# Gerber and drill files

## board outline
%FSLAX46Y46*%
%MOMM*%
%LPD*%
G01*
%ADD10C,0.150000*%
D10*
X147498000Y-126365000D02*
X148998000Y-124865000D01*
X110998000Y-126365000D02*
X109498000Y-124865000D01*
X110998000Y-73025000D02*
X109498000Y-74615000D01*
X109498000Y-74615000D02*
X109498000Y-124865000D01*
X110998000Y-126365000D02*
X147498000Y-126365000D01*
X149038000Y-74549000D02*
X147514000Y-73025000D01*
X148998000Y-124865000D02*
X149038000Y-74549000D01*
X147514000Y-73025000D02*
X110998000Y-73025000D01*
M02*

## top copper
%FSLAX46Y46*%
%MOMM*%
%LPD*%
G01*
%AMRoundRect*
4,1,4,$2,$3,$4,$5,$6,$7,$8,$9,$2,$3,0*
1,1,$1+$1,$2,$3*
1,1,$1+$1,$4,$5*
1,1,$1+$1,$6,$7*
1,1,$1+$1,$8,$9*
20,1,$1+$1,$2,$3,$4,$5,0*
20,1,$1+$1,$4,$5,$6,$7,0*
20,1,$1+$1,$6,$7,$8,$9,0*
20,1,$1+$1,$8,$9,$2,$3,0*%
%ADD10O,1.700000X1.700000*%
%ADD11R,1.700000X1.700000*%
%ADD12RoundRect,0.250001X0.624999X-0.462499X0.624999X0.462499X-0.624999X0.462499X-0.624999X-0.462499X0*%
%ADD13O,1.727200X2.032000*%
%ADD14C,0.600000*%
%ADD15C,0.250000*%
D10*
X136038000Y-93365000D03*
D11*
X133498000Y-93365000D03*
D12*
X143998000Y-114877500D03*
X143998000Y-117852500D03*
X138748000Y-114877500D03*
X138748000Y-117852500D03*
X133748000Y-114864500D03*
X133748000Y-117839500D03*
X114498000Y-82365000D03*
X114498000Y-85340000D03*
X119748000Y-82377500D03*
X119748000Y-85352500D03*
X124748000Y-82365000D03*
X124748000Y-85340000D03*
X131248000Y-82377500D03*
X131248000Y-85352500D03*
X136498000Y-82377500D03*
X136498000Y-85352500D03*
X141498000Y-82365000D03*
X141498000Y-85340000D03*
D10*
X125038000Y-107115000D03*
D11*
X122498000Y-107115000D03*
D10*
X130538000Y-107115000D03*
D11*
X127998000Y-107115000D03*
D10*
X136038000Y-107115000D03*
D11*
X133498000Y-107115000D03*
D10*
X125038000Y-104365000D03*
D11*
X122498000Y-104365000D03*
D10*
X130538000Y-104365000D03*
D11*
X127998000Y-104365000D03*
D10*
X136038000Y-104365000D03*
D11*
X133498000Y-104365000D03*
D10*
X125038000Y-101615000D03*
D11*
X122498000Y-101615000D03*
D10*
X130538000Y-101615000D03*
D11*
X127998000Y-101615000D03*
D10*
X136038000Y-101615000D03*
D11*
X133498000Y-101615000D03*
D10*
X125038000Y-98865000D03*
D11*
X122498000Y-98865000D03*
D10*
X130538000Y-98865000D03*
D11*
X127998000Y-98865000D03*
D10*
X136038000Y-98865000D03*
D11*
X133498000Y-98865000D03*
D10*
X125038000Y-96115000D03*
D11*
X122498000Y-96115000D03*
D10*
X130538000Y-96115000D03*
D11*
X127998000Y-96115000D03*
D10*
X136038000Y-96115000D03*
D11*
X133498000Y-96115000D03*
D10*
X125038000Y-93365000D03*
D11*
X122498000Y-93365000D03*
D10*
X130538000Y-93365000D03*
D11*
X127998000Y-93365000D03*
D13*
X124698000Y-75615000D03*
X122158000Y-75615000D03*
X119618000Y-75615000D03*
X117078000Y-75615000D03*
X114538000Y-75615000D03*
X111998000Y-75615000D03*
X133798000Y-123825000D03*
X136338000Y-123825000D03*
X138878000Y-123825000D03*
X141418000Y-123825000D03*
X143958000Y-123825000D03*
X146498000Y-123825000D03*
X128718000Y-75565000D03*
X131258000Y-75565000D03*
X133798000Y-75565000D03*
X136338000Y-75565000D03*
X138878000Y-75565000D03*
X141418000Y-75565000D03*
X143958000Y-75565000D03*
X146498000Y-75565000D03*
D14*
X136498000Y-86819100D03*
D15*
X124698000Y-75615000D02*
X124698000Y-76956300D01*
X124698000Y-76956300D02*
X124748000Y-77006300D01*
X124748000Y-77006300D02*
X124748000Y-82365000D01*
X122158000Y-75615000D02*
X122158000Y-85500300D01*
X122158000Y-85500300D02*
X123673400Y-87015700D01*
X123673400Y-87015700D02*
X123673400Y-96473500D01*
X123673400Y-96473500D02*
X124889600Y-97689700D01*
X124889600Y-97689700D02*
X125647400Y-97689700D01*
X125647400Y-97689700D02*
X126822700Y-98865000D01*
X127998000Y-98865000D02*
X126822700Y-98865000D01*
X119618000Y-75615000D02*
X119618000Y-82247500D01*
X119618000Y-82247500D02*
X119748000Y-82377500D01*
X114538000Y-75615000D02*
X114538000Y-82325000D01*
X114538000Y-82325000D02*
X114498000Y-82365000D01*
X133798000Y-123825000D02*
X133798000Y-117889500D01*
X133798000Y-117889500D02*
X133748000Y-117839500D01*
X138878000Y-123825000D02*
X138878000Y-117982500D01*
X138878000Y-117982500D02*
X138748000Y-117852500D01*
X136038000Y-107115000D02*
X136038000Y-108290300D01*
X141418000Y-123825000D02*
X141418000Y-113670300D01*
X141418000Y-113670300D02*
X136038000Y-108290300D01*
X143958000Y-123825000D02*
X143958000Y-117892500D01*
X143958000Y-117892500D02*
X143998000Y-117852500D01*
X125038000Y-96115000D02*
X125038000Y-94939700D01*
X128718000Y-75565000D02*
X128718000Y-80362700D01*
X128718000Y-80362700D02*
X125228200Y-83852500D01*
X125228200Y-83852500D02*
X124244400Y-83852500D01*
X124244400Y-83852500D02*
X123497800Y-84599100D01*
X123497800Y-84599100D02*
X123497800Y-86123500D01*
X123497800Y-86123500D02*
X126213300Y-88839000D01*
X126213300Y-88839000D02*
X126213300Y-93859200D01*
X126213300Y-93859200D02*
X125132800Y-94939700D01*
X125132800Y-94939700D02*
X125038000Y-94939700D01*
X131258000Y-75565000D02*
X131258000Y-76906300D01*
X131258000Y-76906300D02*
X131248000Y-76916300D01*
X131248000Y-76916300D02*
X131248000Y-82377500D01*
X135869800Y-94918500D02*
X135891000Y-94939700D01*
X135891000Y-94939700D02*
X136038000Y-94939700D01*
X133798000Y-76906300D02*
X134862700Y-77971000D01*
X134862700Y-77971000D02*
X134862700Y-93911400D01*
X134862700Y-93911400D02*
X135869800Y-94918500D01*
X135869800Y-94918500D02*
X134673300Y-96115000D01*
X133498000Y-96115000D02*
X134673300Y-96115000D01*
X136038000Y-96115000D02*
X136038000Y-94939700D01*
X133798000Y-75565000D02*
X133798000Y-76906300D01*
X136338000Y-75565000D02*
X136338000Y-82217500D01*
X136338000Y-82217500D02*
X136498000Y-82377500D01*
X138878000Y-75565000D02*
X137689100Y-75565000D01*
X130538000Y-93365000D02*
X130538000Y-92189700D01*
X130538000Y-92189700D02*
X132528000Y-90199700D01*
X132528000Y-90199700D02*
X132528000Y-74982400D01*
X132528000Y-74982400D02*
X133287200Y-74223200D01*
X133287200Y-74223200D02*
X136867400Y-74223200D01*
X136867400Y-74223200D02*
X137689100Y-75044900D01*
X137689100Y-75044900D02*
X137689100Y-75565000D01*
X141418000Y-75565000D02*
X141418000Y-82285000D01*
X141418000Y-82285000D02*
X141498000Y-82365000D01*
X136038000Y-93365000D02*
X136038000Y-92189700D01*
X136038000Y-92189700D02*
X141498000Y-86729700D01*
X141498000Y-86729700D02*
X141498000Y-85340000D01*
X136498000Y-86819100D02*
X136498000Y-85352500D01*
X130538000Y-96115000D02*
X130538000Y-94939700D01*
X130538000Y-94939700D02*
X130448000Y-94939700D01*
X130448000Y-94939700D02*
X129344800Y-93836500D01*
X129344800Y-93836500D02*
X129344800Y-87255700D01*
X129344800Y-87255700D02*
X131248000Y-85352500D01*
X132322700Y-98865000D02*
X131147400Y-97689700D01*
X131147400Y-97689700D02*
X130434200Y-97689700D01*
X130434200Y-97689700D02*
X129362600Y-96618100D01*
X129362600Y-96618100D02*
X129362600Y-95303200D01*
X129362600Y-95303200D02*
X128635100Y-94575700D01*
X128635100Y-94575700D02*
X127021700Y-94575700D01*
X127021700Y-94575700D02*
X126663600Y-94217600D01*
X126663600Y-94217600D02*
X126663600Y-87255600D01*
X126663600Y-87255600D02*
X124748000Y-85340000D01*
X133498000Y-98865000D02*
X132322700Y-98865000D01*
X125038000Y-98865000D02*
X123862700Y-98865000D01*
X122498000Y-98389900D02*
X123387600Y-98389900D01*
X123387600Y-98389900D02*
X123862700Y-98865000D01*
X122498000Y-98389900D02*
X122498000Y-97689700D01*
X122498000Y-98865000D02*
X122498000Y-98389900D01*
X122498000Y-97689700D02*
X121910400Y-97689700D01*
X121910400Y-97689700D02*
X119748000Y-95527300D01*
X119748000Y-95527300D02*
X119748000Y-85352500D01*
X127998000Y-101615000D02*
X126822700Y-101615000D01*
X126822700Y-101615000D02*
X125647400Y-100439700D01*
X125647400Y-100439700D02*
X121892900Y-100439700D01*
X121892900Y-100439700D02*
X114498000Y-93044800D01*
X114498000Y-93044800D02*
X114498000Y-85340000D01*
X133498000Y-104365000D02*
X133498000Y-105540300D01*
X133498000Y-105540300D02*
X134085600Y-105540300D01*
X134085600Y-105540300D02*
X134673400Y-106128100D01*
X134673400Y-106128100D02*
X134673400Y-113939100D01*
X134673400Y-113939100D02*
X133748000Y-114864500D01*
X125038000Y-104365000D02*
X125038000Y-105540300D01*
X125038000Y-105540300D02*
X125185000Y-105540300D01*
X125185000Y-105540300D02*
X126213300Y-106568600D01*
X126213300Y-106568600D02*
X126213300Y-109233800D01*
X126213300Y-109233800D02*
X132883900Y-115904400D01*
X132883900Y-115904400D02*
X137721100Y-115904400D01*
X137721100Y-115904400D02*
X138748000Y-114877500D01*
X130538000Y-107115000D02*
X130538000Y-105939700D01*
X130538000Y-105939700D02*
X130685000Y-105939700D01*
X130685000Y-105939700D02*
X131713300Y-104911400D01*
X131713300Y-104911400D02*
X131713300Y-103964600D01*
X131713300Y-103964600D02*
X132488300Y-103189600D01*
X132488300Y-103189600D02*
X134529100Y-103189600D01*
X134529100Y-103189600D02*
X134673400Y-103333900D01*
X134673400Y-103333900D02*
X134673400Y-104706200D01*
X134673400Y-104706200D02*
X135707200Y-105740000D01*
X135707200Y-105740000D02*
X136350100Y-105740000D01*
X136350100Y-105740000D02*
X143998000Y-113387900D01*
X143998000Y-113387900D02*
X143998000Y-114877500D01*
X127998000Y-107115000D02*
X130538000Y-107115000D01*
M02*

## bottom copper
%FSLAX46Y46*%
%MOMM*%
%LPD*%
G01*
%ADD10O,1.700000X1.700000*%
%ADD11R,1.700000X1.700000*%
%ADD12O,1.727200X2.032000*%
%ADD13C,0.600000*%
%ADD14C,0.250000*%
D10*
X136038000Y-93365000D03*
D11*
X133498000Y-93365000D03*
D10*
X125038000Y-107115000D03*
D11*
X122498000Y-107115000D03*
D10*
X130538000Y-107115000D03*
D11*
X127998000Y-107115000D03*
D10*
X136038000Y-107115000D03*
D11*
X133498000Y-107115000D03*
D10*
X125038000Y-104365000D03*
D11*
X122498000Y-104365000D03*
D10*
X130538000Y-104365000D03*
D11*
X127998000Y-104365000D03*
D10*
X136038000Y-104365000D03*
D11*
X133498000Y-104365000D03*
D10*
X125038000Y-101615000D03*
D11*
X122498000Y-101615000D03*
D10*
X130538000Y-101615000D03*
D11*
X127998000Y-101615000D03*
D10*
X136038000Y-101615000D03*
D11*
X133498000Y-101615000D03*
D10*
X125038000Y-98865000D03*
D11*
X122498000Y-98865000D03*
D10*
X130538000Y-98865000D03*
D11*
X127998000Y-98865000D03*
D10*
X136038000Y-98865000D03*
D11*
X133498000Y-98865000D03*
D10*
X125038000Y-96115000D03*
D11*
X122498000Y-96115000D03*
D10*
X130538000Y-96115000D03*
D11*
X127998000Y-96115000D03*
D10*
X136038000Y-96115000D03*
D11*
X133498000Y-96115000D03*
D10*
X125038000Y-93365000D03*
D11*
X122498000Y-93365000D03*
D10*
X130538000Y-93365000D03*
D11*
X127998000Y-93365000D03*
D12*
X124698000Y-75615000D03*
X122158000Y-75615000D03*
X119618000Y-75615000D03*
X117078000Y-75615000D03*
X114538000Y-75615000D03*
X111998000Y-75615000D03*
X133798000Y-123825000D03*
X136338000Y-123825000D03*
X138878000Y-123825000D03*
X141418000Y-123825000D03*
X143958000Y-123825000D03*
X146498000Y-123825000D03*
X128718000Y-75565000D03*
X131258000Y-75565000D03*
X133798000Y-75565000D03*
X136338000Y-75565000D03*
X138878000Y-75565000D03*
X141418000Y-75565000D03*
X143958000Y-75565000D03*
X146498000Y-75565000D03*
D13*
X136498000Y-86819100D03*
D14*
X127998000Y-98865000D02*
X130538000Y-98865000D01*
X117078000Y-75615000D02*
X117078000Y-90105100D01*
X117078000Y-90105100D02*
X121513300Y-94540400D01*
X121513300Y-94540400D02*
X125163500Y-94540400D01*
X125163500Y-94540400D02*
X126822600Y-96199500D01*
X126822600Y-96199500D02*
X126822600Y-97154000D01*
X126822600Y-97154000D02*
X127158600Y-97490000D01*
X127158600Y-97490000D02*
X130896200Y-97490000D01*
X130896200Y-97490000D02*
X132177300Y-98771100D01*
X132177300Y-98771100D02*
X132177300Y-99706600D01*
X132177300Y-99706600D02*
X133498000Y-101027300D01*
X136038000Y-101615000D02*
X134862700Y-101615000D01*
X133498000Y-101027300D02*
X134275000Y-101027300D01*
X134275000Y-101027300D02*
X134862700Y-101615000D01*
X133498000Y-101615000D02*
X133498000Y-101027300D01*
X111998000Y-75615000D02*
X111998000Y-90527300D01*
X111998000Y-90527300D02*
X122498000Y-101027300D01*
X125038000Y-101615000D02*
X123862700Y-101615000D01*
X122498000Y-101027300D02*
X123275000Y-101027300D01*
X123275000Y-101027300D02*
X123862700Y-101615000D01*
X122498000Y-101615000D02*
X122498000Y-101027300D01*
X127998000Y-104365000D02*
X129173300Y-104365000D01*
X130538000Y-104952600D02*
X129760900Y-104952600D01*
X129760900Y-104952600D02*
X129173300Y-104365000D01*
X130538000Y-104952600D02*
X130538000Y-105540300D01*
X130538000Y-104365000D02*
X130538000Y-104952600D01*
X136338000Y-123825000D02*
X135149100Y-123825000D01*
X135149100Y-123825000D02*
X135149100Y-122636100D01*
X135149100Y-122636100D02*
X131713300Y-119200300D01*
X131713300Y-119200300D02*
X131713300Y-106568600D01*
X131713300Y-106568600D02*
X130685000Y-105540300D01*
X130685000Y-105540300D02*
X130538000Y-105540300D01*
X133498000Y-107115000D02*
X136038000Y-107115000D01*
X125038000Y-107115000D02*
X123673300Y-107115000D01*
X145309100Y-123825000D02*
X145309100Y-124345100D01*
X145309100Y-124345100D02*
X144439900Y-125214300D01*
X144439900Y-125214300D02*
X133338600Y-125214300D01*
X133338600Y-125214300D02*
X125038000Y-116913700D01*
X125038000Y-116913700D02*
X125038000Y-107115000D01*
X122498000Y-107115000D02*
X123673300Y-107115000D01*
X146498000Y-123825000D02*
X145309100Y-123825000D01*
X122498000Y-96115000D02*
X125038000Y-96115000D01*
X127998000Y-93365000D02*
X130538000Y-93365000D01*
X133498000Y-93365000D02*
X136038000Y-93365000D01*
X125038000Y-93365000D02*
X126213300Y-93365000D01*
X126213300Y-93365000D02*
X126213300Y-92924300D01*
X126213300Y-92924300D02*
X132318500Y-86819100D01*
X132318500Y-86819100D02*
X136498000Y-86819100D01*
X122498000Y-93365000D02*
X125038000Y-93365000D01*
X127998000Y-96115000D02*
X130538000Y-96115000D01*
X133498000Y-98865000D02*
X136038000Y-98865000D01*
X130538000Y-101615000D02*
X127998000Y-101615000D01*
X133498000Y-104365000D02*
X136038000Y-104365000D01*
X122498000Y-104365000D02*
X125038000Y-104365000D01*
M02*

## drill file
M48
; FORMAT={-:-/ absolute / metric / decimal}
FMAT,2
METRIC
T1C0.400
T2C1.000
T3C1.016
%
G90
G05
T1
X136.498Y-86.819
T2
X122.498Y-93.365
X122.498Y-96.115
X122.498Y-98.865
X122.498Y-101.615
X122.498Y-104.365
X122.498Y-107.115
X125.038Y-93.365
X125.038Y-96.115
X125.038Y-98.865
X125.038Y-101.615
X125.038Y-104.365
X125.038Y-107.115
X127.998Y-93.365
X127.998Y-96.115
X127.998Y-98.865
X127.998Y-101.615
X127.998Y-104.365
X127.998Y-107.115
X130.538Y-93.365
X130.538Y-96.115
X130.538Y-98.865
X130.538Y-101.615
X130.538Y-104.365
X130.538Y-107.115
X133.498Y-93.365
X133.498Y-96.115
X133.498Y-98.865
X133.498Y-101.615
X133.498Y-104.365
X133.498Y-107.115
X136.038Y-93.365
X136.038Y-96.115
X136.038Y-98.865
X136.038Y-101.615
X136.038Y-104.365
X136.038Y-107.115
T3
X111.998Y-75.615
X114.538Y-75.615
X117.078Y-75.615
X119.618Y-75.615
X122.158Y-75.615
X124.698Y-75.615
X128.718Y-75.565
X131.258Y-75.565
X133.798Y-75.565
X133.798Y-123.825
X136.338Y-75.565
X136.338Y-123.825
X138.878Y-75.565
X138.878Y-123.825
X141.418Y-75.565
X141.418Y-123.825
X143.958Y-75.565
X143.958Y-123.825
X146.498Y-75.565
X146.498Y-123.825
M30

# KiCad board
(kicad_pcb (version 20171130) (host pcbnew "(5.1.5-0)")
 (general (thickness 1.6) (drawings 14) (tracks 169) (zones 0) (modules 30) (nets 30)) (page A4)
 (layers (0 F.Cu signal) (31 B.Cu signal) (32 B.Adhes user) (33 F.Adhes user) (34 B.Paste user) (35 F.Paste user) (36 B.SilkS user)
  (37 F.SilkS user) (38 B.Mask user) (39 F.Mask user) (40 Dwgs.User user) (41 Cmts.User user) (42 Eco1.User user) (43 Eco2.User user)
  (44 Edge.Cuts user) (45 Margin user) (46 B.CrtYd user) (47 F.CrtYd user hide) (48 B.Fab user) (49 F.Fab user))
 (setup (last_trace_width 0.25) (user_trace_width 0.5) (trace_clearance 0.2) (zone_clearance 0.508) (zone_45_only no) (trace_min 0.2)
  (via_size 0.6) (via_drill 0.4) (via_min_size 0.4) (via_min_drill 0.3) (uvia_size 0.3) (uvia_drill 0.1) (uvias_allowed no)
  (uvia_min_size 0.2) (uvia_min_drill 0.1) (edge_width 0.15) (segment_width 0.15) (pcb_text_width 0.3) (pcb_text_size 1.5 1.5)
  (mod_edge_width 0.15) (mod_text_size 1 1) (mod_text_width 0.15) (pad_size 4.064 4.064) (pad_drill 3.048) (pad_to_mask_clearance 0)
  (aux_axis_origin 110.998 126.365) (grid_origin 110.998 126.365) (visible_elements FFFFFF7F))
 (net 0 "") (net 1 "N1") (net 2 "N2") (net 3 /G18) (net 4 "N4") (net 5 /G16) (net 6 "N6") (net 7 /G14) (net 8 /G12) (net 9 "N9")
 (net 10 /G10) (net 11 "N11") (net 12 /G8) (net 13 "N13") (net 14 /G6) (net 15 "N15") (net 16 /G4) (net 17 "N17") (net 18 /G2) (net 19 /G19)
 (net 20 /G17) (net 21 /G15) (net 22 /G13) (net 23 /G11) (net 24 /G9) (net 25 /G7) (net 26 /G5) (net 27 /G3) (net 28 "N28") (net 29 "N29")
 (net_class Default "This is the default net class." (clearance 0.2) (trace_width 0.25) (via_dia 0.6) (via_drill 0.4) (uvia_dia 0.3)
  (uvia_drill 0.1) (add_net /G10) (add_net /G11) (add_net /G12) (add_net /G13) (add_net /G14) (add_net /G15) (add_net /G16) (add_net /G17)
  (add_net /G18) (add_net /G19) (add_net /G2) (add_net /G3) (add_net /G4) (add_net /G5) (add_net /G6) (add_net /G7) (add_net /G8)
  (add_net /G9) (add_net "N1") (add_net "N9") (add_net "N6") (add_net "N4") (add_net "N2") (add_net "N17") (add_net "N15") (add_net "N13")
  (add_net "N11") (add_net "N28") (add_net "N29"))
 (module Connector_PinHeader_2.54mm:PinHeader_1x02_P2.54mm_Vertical (layer F.Cu) (at 133.498 93.365 90)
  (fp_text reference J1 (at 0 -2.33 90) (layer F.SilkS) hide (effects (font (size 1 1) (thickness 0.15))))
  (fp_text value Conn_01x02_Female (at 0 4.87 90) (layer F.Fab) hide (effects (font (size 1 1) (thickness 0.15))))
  (pad 2 thru_hole oval (at 0 2.54 90) (size 1.7 1.7) (drill 1) (layers *.Cu *.Mask) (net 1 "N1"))
  (pad 1 thru_hole rect (at 0 0 90) (size 1.7 1.7) (drill 1) (layers *.Cu *.Mask) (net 1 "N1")))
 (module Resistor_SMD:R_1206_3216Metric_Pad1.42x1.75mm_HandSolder (layer F.Cu) (at 143.998 116.365 90)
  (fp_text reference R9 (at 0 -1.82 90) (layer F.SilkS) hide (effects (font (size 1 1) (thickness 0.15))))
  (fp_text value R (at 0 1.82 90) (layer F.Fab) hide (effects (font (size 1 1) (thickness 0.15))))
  (pad 2 smd roundrect (at 1.4875 0 90) (size 1.425 1.75) (layers F.Cu F.Paste F.Mask) (roundrect_rratio 0.175439) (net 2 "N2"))
  (pad 1 smd roundrect (at -1.4875 0 90) (size 1.425 1.75) (layers F.Cu F.Paste F.Mask) (roundrect_rratio 0.175439) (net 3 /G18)))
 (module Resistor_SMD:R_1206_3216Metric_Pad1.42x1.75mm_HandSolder (layer F.Cu) (at 138.748 116.365 90)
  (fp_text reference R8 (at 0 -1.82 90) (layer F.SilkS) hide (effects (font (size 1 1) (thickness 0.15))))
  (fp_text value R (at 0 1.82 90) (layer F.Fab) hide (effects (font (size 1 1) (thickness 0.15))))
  (pad 2 smd roundrect (at 1.4875 0 90) (size 1.425 1.75) (layers F.Cu F.Paste F.Mask) (roundrect_rratio 0.175439) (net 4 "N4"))
  (pad 1 smd roundrect (at -1.4875 0 90) (size 1.425 1.75) (layers F.Cu F.Paste F.Mask) (roundrect_rratio 0.175439) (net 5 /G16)))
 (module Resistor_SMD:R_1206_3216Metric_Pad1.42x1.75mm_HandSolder (layer F.Cu) (at 133.748 116.352 90)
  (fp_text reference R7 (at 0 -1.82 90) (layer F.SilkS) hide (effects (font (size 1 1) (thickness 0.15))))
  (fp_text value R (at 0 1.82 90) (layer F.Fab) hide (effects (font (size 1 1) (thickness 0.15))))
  (pad 2 smd roundrect (at 1.4875 0 90) (size 1.425 1.75) (layers F.Cu F.Paste F.Mask) (roundrect_rratio 0.175439) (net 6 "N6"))
  (pad 1 smd roundrect (at -1.4875 0 90) (size 1.425 1.75) (layers F.Cu F.Paste F.Mask) (roundrect_rratio 0.175439) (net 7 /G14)))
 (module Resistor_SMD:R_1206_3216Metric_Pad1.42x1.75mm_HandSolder (layer F.Cu) (at 114.498 83.8525 90)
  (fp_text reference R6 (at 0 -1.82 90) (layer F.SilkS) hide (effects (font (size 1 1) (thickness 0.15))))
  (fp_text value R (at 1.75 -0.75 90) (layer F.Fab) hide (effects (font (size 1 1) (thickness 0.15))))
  (pad 2 smd roundrect (at 1.4875 0 90) (size 1.425 1.75) (layers F.Cu F.Paste F.Mask) (roundrect_rratio 0.175439) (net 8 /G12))
  (pad 1 smd roundrect (at -1.4875 0 90) (size 1.425 1.75) (layers F.Cu F.Paste F.Mask) (roundrect_rratio 0.175439) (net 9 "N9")))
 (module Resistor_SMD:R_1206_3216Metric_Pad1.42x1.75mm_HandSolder (layer F.Cu) (at 119.748 83.865 90)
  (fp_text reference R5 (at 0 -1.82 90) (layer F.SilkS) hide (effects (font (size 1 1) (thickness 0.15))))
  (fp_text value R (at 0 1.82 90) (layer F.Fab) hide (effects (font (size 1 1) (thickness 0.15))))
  (pad 2 smd roundrect (at 1.4875 0 90) (size 1.425 1.75) (layers F.Cu F.Paste F.Mask) (roundrect_rratio 0.175439) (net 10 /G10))
  (pad 1 smd roundrect (at -1.4875 0 90) (size 1.425 1.75) (layers F.Cu F.Paste F.Mask) (roundrect_rratio 0.175439) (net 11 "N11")))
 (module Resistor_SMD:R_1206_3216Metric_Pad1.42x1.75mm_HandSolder (layer F.Cu) (at 124.748 83.8525 90)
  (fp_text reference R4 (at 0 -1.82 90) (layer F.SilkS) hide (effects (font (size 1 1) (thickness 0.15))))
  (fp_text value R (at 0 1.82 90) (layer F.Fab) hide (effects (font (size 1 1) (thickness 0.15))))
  (pad 2 smd roundrect (at 1.4875 0 90) (size 1.425 1.75) (layers F.Cu F.Paste F.Mask) (roundrect_rratio 0.175439) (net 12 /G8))
  (pad 1 smd roundrect (at -1.4875 0 90) (size 1.425 1.75) (layers F.Cu F.Paste F.Mask) (roundrect_rratio 0.175439) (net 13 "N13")))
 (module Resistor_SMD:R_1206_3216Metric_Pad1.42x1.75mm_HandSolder (layer F.Cu) (at 131.248 83.865 90)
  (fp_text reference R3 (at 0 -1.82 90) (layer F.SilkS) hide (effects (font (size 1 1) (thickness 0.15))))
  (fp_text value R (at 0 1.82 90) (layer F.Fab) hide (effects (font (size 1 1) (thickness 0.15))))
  (pad 2 smd roundrect (at 1.4875 0 90) (size 1.425 1.75) (layers F.Cu F.Paste F.Mask) (roundrect_rratio 0.175439) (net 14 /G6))
  (pad 1 smd roundrect (at -1.4875 0 90) (size 1.425 1.75) (layers F.Cu F.Paste F.Mask) (roundrect_rratio 0.175439) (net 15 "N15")))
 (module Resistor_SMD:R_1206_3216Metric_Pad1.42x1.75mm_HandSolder (layer F.Cu) (at 136.498 83.865 90)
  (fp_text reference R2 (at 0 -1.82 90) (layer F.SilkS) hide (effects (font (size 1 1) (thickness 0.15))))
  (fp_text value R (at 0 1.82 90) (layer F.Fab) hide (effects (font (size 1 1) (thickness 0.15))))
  (pad 2 smd roundrect (at 1.4875 0 90) (size 1.425 1.75) (layers F.Cu F.Paste F.Mask) (roundrect_rratio 0.175439) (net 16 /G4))
  (pad 1 smd roundrect (at -1.4875 0 90) (size 1.425 1.75) (layers F.Cu F.Paste F.Mask) (roundrect_rratio 0.175439) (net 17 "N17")))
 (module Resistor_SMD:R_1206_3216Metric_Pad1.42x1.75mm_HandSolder (layer F.Cu) (at 141.498 83.8525 90)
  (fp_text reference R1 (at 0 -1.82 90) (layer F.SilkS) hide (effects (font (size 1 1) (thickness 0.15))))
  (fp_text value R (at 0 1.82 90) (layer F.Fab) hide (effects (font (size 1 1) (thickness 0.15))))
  (pad 2 smd roundrect (at 1.4875 0 90) (size 1.425 1.75) (layers F.Cu F.Paste F.Mask) (roundrect_rratio 0.175439) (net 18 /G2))
  (pad 1 smd roundrect (at -1.4875 0 90) (size 1.425 1.75) (layers F.Cu F.Paste F.Mask) (roundrect_rratio 0.175439) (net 1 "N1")))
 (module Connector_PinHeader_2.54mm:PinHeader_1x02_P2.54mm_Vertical (layer F.Cu) (at 122.498 107.115 90)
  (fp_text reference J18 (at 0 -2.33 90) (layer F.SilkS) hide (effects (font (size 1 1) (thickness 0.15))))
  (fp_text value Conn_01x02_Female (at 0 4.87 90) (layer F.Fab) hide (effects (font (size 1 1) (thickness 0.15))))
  (pad 2 thru_hole oval (at 0 2.54 90) (size 1.7 1.7) (drill 1) (layers *.Cu *.Mask) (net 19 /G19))
  (pad 1 thru_hole rect (at 0 0 90) (size 1.7 1.7) (drill 1) (layers *.Cu *.Mask) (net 19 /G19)))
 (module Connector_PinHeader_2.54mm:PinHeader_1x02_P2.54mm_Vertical (layer F.Cu) (at 127.998 107.115 90)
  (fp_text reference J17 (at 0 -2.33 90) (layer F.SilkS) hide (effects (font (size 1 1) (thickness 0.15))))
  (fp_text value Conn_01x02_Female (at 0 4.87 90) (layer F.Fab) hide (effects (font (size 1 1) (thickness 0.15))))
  (pad 2 thru_hole oval (at 0 2.54 90) (size 1.7 1.7) (drill 1) (layers *.Cu *.Mask) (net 2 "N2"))
  (pad 1 thru_hole rect (at 0 0 90) (size 1.7 1.7) (drill 1) (layers *.Cu *.Mask) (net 2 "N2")))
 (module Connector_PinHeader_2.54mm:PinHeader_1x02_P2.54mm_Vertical (layer F.Cu) (at 133.498 107.115 90)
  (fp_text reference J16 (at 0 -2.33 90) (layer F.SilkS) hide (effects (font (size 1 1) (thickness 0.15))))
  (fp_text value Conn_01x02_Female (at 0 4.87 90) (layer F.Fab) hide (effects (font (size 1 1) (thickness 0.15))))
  (pad 2 thru_hole oval (at 0 2.54 90) (size 1.7 1.7) (drill 1) (layers *.Cu *.Mask) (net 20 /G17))
  (pad 1 thru_hole rect (at 0 0 90) (size 1.7 1.7) (drill 1) (layers *.Cu *.Mask) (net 20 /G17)))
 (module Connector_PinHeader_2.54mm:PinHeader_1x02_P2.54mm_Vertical (layer F.Cu) (at 122.498 104.365 90)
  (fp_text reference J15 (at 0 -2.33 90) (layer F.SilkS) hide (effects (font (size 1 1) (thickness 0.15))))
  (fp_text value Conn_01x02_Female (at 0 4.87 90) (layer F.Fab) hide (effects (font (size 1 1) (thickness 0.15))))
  (pad 2 thru_hole oval (at 0 2.54 90) (size 1.7 1.7) (drill 1) (layers *.Cu *.Mask) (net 4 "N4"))
  (pad 1 thru_hole rect (at 0 0 90) (size 1.7 1.7) (drill 1) (layers *.Cu *.Mask) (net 4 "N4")))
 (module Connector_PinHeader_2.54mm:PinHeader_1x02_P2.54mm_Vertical (layer F.Cu) (at 127.998 104.365 90)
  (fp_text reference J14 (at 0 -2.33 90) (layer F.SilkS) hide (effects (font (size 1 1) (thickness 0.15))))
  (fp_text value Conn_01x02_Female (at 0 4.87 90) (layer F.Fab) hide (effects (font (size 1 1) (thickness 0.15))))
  (pad 2 thru_hole oval (at 0 2.54 90) (size 1.7 1.7) (drill 1) (layers *.Cu *.Mask) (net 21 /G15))
  (pad 1 thru_hole rect (at 0 0 90) (size 1.7 1.7) (drill 1) (layers *.Cu *.Mask) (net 21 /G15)))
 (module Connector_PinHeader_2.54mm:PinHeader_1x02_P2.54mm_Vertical (layer F.Cu) (at 133.498 104.365 90)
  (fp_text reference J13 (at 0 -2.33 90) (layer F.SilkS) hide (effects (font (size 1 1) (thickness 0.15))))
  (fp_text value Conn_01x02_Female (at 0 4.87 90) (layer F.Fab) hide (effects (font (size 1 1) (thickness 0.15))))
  (pad 2 thru_hole oval (at 0 2.54 90) (size 1.7 1.7) (drill 1) (layers *.Cu *.Mask) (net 6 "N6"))
  (pad 1 thru_hole rect (at 0 0 90) (size 1.7 1.7) (drill 1) (layers *.Cu *.Mask) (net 6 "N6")))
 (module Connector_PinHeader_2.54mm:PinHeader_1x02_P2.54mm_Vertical (layer F.Cu) (at 122.498 101.615 90)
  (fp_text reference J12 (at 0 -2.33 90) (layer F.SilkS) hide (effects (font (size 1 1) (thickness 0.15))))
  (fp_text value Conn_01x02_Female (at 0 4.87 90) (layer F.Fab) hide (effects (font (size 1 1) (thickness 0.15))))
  (pad 2 thru_hole oval (at 0 2.54 90) (size 1.7 1.7) (drill 1) (layers *.Cu *.Mask) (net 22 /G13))
  (pad 1 thru_hole rect (at 0 0 90) (size 1.7 1.7) (drill 1) (layers *.Cu *.Mask) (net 22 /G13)))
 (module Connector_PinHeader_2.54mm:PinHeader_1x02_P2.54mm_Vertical (layer F.Cu) (at 127.998 101.615 90)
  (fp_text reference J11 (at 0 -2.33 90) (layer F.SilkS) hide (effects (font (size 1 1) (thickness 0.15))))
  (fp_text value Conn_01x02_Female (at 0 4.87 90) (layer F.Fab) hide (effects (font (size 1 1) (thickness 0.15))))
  (pad 2 thru_hole oval (at 0 2.54 90) (size 1.7 1.7) (drill 1) (layers *.Cu *.Mask) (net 9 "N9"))
  (pad 1 thru_hole rect (at 0 0 90) (size 1.7 1.7) (drill 1) (layers *.Cu *.Mask) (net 9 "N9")))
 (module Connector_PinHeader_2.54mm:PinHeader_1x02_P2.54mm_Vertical (layer F.Cu) (at 133.498 101.615 90)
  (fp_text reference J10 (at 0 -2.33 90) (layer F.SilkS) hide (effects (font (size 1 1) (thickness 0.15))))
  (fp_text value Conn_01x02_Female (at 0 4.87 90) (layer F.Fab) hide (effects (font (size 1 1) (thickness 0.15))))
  (pad 2 thru_hole oval (at 0 2.54 90) (size 1.7 1.7) (drill 1) (layers *.Cu *.Mask) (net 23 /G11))
  (pad 1 thru_hole rect (at 0 0 90) (size 1.7 1.7) (drill 1) (layers *.Cu *.Mask) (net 23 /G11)))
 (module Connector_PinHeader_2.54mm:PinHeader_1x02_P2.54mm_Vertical (layer F.Cu) (at 122.498 98.865 90)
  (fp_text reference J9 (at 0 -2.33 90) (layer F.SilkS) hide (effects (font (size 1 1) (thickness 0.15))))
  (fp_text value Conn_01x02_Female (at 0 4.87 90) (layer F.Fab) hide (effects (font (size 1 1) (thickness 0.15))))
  (pad 2 thru_hole oval (at 0 2.54 90) (size 1.7 1.7) (drill 1) (layers *.Cu *.Mask) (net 11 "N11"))
  (pad 1 thru_hole rect (at 0 0 90) (size 1.7 1.7) (drill 1) (layers *.Cu *.Mask) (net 11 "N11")))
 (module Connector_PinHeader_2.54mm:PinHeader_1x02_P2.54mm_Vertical (layer F.Cu) (at 127.998 98.865 90)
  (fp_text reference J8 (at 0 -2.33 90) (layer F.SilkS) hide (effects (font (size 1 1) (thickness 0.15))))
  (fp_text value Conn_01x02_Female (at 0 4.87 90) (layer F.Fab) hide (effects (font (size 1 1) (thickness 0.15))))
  (pad 2 thru_hole oval (at 0 2.54 90) (size 1.7 1.7) (drill 1) (layers *.Cu *.Mask) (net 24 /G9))
  (pad 1 thru_hole rect (at 0 0 90) (size 1.7 1.7) (drill 1) (layers *.Cu *.Mask) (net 24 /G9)))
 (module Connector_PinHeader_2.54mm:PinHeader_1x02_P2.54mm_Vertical (layer F.Cu) (at 133.498 98.865 90)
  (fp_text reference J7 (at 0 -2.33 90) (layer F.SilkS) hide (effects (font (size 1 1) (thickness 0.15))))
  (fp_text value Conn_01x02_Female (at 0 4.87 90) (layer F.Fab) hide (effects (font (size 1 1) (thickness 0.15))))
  (pad 2 thru_hole oval (at 0 2.54 90) (size 1.7 1.7) (drill 1) (layers *.Cu *.Mask) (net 13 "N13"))
  (pad 1 thru_hole rect (at 0 0 90) (size 1.7 1.7) (drill 1) (layers *.Cu *.Mask) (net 13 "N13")))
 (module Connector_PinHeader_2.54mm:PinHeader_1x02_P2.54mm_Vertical (layer F.Cu) (at 122.498 96.115 90)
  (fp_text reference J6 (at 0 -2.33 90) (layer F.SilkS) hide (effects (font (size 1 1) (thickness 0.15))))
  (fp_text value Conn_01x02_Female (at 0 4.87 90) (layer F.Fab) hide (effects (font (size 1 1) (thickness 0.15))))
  (pad 2 thru_hole oval (at 0 2.54 90) (size 1.7 1.7) (drill 1) (layers *.Cu *.Mask) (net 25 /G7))
  (pad 1 thru_hole rect (at 0 0 90) (size 1.7 1.7) (drill 1) (layers *.Cu *.Mask) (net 25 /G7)))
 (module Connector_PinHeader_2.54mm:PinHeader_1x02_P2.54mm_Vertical (layer F.Cu) (at 127.998 96.115 90)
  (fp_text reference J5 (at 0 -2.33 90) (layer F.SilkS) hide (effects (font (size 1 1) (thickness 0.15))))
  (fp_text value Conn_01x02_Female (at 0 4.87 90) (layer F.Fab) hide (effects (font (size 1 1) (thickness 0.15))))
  (pad 2 thru_hole oval (at 0 2.54 90) (size 1.7 1.7) (drill 1) (layers *.Cu *.Mask) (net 15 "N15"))
  (pad 1 thru_hole rect (at 0 0 90) (size 1.7 1.7) (drill 1) (layers *.Cu *.Mask) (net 15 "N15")))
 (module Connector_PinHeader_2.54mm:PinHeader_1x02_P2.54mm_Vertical (layer F.Cu) (at 133.498 96.115 90)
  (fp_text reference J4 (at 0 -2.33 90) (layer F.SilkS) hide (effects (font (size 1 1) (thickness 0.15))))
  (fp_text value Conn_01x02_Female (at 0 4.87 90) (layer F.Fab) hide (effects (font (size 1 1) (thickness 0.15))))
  (pad 2 thru_hole oval (at 0 2.54 90) (size 1.7 1.7) (drill 1) (layers *.Cu *.Mask) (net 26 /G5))
  (pad 1 thru_hole rect (at 0 0 90) (size 1.7 1.7) (drill 1) (layers *.Cu *.Mask) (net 26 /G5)))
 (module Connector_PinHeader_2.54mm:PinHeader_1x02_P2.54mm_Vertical (layer F.Cu) (at 122.498 93.365 90)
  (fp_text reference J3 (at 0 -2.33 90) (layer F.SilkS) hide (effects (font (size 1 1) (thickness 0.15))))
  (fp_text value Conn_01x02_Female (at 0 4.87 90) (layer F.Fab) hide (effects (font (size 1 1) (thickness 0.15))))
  (pad 2 thru_hole oval (at 0 2.54 90) (size 1.7 1.7) (drill 1) (layers *.Cu *.Mask) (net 17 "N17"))
  (pad 1 thru_hole rect (at 0 0 90) (size 1.7 1.7) (drill 1) (layers *.Cu *.Mask) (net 17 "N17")))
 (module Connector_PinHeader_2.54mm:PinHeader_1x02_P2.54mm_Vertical (layer F.Cu) (at 127.998 93.365 90)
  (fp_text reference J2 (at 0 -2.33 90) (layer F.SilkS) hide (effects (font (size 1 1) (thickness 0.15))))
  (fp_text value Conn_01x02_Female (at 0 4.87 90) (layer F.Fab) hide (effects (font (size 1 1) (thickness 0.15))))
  (pad 2 thru_hole oval (at 0 2.54 90) (size 1.7 1.7) (drill 1) (layers *.Cu *.Mask) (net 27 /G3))
  (pad 1 thru_hole rect (at 0 0 90) (size 1.7 1.7) (drill 1) (layers *.Cu *.Mask) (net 27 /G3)))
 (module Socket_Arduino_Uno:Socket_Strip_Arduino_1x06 (layer F.Cu) (at 111.998 75.615)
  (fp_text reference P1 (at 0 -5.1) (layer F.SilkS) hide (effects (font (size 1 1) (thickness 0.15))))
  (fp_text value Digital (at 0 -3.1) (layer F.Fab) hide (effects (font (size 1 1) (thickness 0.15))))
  (pad 6 thru_hole oval (at 12.7 0) (size 1.7272 2.032) (drill 1.016) (layers *.Cu *.Mask F.SilkS) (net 12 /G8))
  (pad 5 thru_hole oval (at 10.16 0) (size 1.7272 2.032) (drill 1.016) (layers *.Cu *.Mask F.SilkS) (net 24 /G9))
  (pad 4 thru_hole oval (at 7.62 0) (size 1.7272 2.032) (drill 1.016) (layers *.Cu *.Mask F.SilkS) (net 10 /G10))
  (pad 3 thru_hole oval (at 5.08 0) (size 1.7272 2.032) (drill 1.016) (layers *.Cu *.Mask F.SilkS) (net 23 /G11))
  (pad 2 thru_hole oval (at 2.54 0) (size 1.7272 2.032) (drill 1.016) (layers *.Cu *.Mask F.SilkS) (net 8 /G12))
  (pad 1 thru_hole oval (at 0 0) (size 1.7272 2.032) (drill 1.016) (layers *.Cu *.Mask F.SilkS) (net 22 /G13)))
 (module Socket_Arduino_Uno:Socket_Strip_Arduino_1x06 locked (layer F.Cu) (at 133.798 123.825)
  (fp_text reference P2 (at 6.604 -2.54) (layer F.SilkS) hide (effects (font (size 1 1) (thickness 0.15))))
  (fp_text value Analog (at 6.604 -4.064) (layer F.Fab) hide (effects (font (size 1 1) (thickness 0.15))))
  (pad 1 thru_hole oval (at 0 0) (size 1.7272 2.032) (drill 1.016) (layers *.Cu *.Mask F.SilkS) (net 7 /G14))
  (pad 2 thru_hole oval (at 2.54 0) (size 1.7272 2.032) (drill 1.016) (layers *.Cu *.Mask F.SilkS) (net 21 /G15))
  (pad 3 thru_hole oval (at 5.08 0) (size 1.7272 2.032) (drill 1.016) (layers *.Cu *.Mask F.SilkS) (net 5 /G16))
  (pad 4 thru_hole oval (at 7.62 0) (size 1.7272 2.032) (drill 1.016) (layers *.Cu *.Mask F.SilkS) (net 20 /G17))
  (pad 5 thru_hole oval (at 10.16 0) (size 1.7272 2.032) (drill 1.016) (layers *.Cu *.Mask F.SilkS) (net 3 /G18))
  (pad 6 thru_hole oval (at 12.7 0) (size 1.7272 2.032) (drill 1.016) (layers *.Cu *.Mask F.SilkS) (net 19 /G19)))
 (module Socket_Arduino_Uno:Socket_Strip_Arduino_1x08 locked (layer F.Cu) (at 128.718 75.565)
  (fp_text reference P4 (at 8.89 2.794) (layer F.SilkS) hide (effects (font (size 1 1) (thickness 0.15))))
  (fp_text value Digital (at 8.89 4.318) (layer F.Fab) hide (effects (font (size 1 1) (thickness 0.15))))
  (pad 1 thru_hole oval (at 0 0) (size 1.7272 2.032) (drill 1.016) (layers *.Cu *.Mask F.SilkS) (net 25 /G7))
  (pad 2 thru_hole oval (at 2.54 0) (size 1.7272 2.032) (drill 1.016) (layers *.Cu *.Mask F.SilkS) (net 14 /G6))
  (pad 3 thru_hole oval (at 5.08 0) (size 1.7272 2.032) (drill 1.016) (layers *.Cu *.Mask F.SilkS) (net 26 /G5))
  (pad 4 thru_hole oval (at 7.62 0) (size 1.7272 2.032) (drill 1.016) (layers *.Cu *.Mask F.SilkS) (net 16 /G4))
  (pad 5 thru_hole oval (at 10.16 0) (size 1.7272 2.032) (drill 1.016) (layers *.Cu *.Mask F.SilkS) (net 27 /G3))
  (pad 6 thru_hole oval (at 12.7 0) (size 1.7272 2.032) (drill 1.016) (layers *.Cu *.Mask F.SilkS) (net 18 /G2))
  (pad 7 thru_hole oval (at 15.24 0) (size 1.7272 2.032) (drill 1.016) (layers *.Cu *.Mask F.SilkS) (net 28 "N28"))
  (pad 8 thru_hole oval (at 17.78 0) (size 1.7272 2.032) (drill 1.016) (layers *.Cu *.Mask F.SilkS) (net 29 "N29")))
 (gr_line (start 147.498 126.365) (end 148.998 124.865) (angle 90) (layer Edge.Cuts) (width 0.15))
 (gr_line (start 110.998 126.365) (end 109.498 124.865) (layer Edge.Cuts) (width 0.15))
 (gr_line (start 110.998 73.025) (end 109.498 74.615) (layer Edge.Cuts) (width 0.15))
 (gr_line (start 109.498 74.615) (end 109.498 124.865) (angle 90) (layer Edge.Cuts) (width 0.15))
 (gr_line (start 110.998 126.365) (end 147.498 126.365) (angle 90) (layer Edge.Cuts) (width 0.15))
 (gr_line (start 149.038 74.549) (end 147.514 73.025) (angle 90) (layer Edge.Cuts) (width 0.15))
 (gr_line (start 148.998 124.865) (end 149.038 74.549) (angle 90) (layer Edge.Cuts) (width 0.15))
 (gr_line (start 147.514 73.025) (end 110.998 73.025) (angle 90) (layer Edge.Cuts) (width 0.15))
 (segment (start 124.698 75.615) (end 124.698 76.9563) (width 0.25) (layer F.Cu) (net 12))
 (segment (start 124.698 76.9563) (end 124.748 77.0063) (width 0.25) (layer F.Cu) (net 12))
 (segment (start 124.748 77.0063) (end 124.748 82.365) (width 0.25) (layer F.Cu) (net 12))
 (segment (start 122.158 75.615) (end 122.158 85.5003) (width 0.25) (layer F.Cu) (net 24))
 (segment (start 122.158 85.5003) (end 123.6734 87.0157) (width 0.25) (layer F.Cu) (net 24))
 (segment (start 123.6734 87.0157) (end 123.6734 96.4735) (width 0.25) (layer F.Cu) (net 24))
 (segment (start 123.6734 96.4735) (end 124.8896 97.6897) (width 0.25) (layer F.Cu) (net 24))
 (segment (start 124.8896 97.6897) (end 125.6474 97.6897) (width 0.25) (layer F.Cu) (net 24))
 (segment (start 125.6474 97.6897) (end 126.8227 98.865) (width 0.25) (layer F.Cu) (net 24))
 (segment (start 127.998 98.865) (end 130.538 98.865) (width 0.25) (layer B.Cu) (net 24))
 (segment (start 127.998 98.865) (end 126.8227 98.865) (width 0.25) (layer F.Cu) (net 24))
 (segment (start 119.618 75.615) (end 119.618 82.2475) (width 0.25) (layer F.Cu) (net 10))
 (segment (start 119.618 82.2475) (end 119.748 82.3775) (width 0.25) (layer F.Cu) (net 10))
 (segment (start 117.078 75.615) (end 117.078 90.1051) (width 0.25) (layer B.Cu) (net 23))
 (segment (start 117.078 90.1051) (end 121.5133 94.5404) (width 0.25) (layer B.Cu) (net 23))
 (segment (start 121.5133 94.5404) (end 125.1635 94.5404) (width 0.25) (layer B.Cu) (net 23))
 (segment (start 125.1635 94.5404) (end 126.8226 96.1995) (width 0.25) (layer B.Cu) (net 23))
 (segment (start 126.8226 96.1995) (end 126.8226 97.154) (width 0.25) (layer B.Cu) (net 23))
 (segment (start 126.8226 97.154) (end 127.1586 97.49) (width 0.25) (layer B.Cu) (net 23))
 (segment (start 127.1586 97.49) (end 130.8962 97.49) (width 0.25) (layer B.Cu) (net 23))
 (segment (start 130.8962 97.49) (end 132.1773 98.7711) (width 0.25) (layer B.Cu) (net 23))
 (segment (start 132.1773 98.7711) (end 132.1773 99.7066) (width 0.25) (layer B.Cu) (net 23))
 (segment (start 132.1773 99.7066) (end 133.498 101.0273) (width 0.25) (layer B.Cu) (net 23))
 (segment (start 136.038 101.615) (end 134.8627 101.615) (width 0.25) (layer B.Cu) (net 23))
 (segment (start 133.498 101.0273) (end 134.275 101.0273) (width 0.25) (layer B.Cu) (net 23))
 (segment (start 134.275 101.0273) (end 134.8627 101.615) (width 0.25) (layer B.Cu) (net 23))
 (segment (start 133.498 101.615) (end 133.498 101.0273) (width 0.25) (layer B.Cu) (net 23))
 (segment (start 114.538 75.615) (end 114.538 82.325) (width 0.25) (layer F.Cu) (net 8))
 (segment (start 114.538 82.325) (end 114.498 82.365) (width 0.25) (layer F.Cu) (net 8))
 (segment (start 111.998 75.615) (end 111.998 90.5273) (width 0.25) (layer B.Cu) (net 22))
 (segment (start 111.998 90.5273) (end 122.498 101.0273) (width 0.25) (layer B.Cu) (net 22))
 (segment (start 125.038 101.615) (end 123.8627 101.615) (width 0.25) (layer B.Cu) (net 22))
 (segment (start 122.498 101.0273) (end 123.275 101.0273) (width 0.25) (layer B.Cu) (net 22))
 (segment (start 123.275 101.0273) (end 123.8627 101.615) (width 0.25) (layer B.Cu) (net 22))
 (segment (start 122.498 101.615) (end 122.498 101.0273) (width 0.25) (layer B.Cu) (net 22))
 (segment (start 133.798 123.825) (end 133.798 117.8895) (width 0.25) (layer F.Cu) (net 7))
 (segment (start 133.798 117.8895) (end 133.748 117.8395) (width 0.25) (layer F.Cu) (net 7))
 (segment (start 127.998 104.365) (end 129.1733 104.365) (width 0.25) (layer B.Cu) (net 21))
 (segment (start 130.538 104.9526) (end 129.7609 104.9526) (width 0.25) (layer B.Cu) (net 21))
 (segment (start 129.7609 104.9526) (end 129.1733 104.365) (width 0.25) (layer B.Cu) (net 21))
 (segment (start 130.538 104.9526) (end 130.538 105.5403) (width 0.25) (layer B.Cu) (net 21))
 (segment (start 130.538 104.365) (end 130.538 104.9526) (width 0.25) (layer B.Cu) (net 21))
 (segment (start 136.338 123.825) (end 135.1491 123.825) (width 0.25) (layer B.Cu) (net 21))
 (segment (start 135.1491 123.825) (end 135.1491 122.6361) (width 0.25) (layer B.Cu) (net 21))
 (segment (start 135.1491 122.6361) (end 131.7133 119.2003) (width 0.25) (layer B.Cu) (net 21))
 (segment (start 131.7133 119.2003) (end 131.7133 106.5686) (width 0.25) (layer B.Cu) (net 21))
 (segment (start 131.7133 106.5686) (end 130.685 105.5403) (width 0.25) (layer B.Cu) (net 21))
 (segment (start 130.685 105.5403) (end 130.538 105.5403) (width 0.25) (layer B.Cu) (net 21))
 (segment (start 138.878 123.825) (end 138.878 117.9825) (width 0.25) (layer F.Cu) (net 5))
 (segment (start 138.878 117.9825) (end 138.748 117.8525) (width 0.25) (layer F.Cu) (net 5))
 (segment (start 136.038 107.115) (end 136.038 108.2903) (width 0.25) (layer F.Cu) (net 20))
 (segment (start 141.418 123.825) (end 141.418 113.6703) (width 0.25) (layer F.Cu) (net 20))
 (segment (start 141.418 113.6703) (end 136.038 108.2903) (width 0.25) (layer F.Cu) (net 20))
 (segment (start 133.498 107.115) (end 136.038 107.115) (width 0.25) (layer B.Cu) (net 20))
 (segment (start 143.958 123.825) (end 143.958 117.8925) (width 0.25) (layer F.Cu) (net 3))
 (segment (start 143.958 117.8925) (end 143.998 117.8525) (width 0.25) (layer F.Cu) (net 3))
 (segment (start 125.038 107.115) (end 123.6733 107.115) (width 0.25) (layer B.Cu) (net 19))
 (segment (start 145.3091 123.825) (end 145.3091 124.3451) (width 0.25) (layer B.Cu) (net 19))
 (segment (start 145.3091 124.3451) (end 144.4399 125.2143) (width 0.25) (layer B.Cu) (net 19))
 (segment (start 144.4399 125.2143) (end 133.3386 125.2143) (width 0.25) (layer B.Cu) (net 19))
 (segment (start 133.3386 125.2143) (end 125.038 116.9137) (width 0.25) (layer B.Cu) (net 19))
 (segment (start 125.038 116.9137) (end 125.038 107.115) (width 0.25) (layer B.Cu) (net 19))
 (segment (start 122.498 107.115) (end 123.6733 107.115) (width 0.25) (layer B.Cu) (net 19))
 (segment (start 146.498 123.825) (end 145.3091 123.825) (width 0.25) (layer B.Cu) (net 19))
 (segment (start 125.038 96.115) (end 125.038 94.9397) (width 0.25) (layer F.Cu) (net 25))
 (segment (start 128.718 75.565) (end 128.718 80.3627) (width 0.25) (layer F.Cu) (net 25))
 (segment (start 128.718 80.3627) (end 125.2282 83.8525) (width 0.25) (layer F.Cu) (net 25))
 (segment (start 125.2282 83.8525) (end 124.2444 83.8525) (width 0.25) (layer F.Cu) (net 25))
 (segment (start 124.2444 83.8525) (end 123.4978 84.5991) (width 0.25) (layer F.Cu) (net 25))
 (segment (start 123.4978 84.5991) (end 123.4978 86.1235) (width 0.25) (layer F.Cu) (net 25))
 (segment (start 123.4978 86.1235) (end 126.2133 88.839) (width 0.25) (layer F.Cu) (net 25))
 (segment (start 126.2133 88.839) (end 126.2133 93.8592) (width 0.25) (layer F.Cu) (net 25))
 (segment (start 126.2133 93.8592) (end 125.1328 94.9397) (width 0.25) (layer F.Cu) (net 25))
 (segment (start 125.1328 94.9397) (end 125.038 94.9397) (width 0.25) (layer F.Cu) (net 25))
 (segment (start 122.498 96.115) (end 125.038 96.115) (width 0.25) (layer B.Cu) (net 25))
 (segment (start 131.258 75.565) (end 131.258 76.9063) (width 0.25) (layer F.Cu) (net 14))
 (segment (start 131.258 76.9063) (end 131.248 76.9163) (width 0.25) (layer F.Cu) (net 14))
 (segment (start 131.248 76.9163) (end 131.248 82.3775) (width 0.25) (layer F.Cu) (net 14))
 (segment (start 135.8698 94.9185) (end 135.891 94.9397) (width 0.25) (layer F.Cu) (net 26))
 (segment (start 135.891 94.9397) (end 136.038 94.9397) (width 0.25) (layer F.Cu) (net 26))
 (segment (start 133.798 76.9063) (end 134.8627 77.971) (width 0.25) (layer F.Cu) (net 26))
 (segment (start 134.8627 77.971) (end 134.8627 93.9114) (width 0.25) (layer F.Cu) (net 26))
 (segment (start 134.8627 93.9114) (end 135.8698 94.9185) (width 0.25) (layer F.Cu) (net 26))
 (segment (start 135.8698 94.9185) (end 134.6733 96.115) (width 0.25) (layer F.Cu) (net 26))
 (segment (start 133.498 96.115) (end 134.6733 96.115) (width 0.25) (layer F.Cu) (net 26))
 (segment (start 136.038 96.115) (end 136.038 94.9397) (width 0.25) (layer F.Cu) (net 26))
 (segment (start 133.798 75.565) (end 133.798 76.9063) (width 0.25) (layer F.Cu) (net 26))
 (segment (start 136.338 75.565) (end 136.338 82.2175) (width 0.25) (layer F.Cu) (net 16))
 (segment (start 136.338 82.2175) (end 136.498 82.3775) (width 0.25) (layer F.Cu) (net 16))
 (segment (start 138.878 75.565) (end 137.6891 75.565) (width 0.25) (layer F.Cu) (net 27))
 (segment (start 130.538 93.365) (end 130.538 92.1897) (width 0.25) (layer F.Cu) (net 27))
 (segment (start 130.538 92.1897) (end 132.528 90.1997) (width 0.25) (layer F.Cu) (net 27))
 (segment (start 132.528 90.1997) (end 132.528 74.9824) (width 0.25) (layer F.Cu) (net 27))
 (segment (start 132.528 74.9824) (end 133.2872 74.2232) (width 0.25) (layer F.Cu) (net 27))
 (segment (start 133.2872 74.2232) (end 136.8674 74.2232) (width 0.25) (layer F.Cu) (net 27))
 (segment (start 136.8674 74.2232) (end 137.6891 75.0449) (width 0.25) (layer F.Cu) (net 27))
 (segment (start 137.6891 75.0449) (end 137.6891 75.565) (width 0.25) (layer F.Cu) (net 27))
 (segment (start 127.998 93.365) (end 130.538 93.365) (width 0.25) (layer B.Cu) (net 27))
 (segment (start 141.418 75.565) (end 141.418 82.285) (width 0.25) (layer F.Cu) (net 18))
 (segment (start 141.418 82.285) (end 141.498 82.365) (width 0.25) (layer F.Cu) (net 18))
 (segment (start 136.038 93.365) (end 136.038 92.1897) (width 0.25) (layer F.Cu) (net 1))
 (segment (start 136.038 92.1897) (end 141.498 86.7297) (width 0.25) (layer F.Cu) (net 1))
 (segment (start 141.498 86.7297) (end 141.498 85.34) (width 0.25) (layer F.Cu) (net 1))
 (segment (start 133.498 93.365) (end 136.038 93.365) (width 0.25) (layer B.Cu) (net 1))
 (segment (start 125.038 93.365) (end 126.2133 93.365) (width 0.25) (layer B.Cu) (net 17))
 (segment (start 126.2133 93.365) (end 126.2133 92.9243) (width 0.25) (layer B.Cu) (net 17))
 (segment (start 126.2133 92.9243) (end 132.3185 86.8191) (width 0.25) (layer B.Cu) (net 17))
 (segment (start 132.3185 86.8191) (end 136.498 86.8191) (width 0.25) (layer B.Cu) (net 17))
 (segment (start 122.498 93.365) (end 125.038 93.365) (width 0.25) (layer B.Cu) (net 17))
 (segment (start 136.498 86.8191) (end 136.498 85.3525) (width 0.25) (layer F.Cu) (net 17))
 (via (at 136.498 86.8191) (size 0.6) (layers F.Cu B.Cu) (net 17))
 (segment (start 130.538 96.115) (end 130.538 94.9397) (width 0.25) (layer F.Cu) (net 15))
 (segment (start 130.538 94.9397) (end 130.448 94.9397) (width 0.25) (layer F.Cu) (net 15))
 (segment (start 130.448 94.9397) (end 129.3448 93.8365) (width 0.25) (layer F.Cu) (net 15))
 (segment (start 129.3448 93.8365) (end 129.3448 87.2557) (width 0.25) (layer F.Cu) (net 15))
 (segment (start 129.3448 87.2557) (end 131.248 85.3525) (width 0.25) (layer F.Cu) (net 15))
 (segment (start 127.998 96.115) (end 130.538 96.115) (width 0.25) (layer B.Cu) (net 15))
 (segment (start 132.3227 98.865) (end 131.1474 97.6897) (width 0.25) (layer F.Cu) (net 13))
 (segment (start 131.1474 97.6897) (end 130.4342 97.6897) (width 0.25) (layer F.Cu) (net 13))
 (segment (start 130.4342 97.6897) (end 129.3626 96.6181) (width 0.25) (layer F.Cu) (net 13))
 (segment (start 129.3626 96.6181) (end 129.3626 95.3032) (width 0.25) (layer F.Cu) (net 13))
 (segment (start 129.3626 95.3032) (end 128.6351 94.5757) (width 0.25) (layer F.Cu) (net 13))
 (segment (start 128.6351 94.5757) (end 127.0217 94.5757) (width 0.25) (layer F.Cu) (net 13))
 (segment (start 127.0217 94.5757) (end 126.6636 94.2176) (width 0.25) (layer F.Cu) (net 13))
 (segment (start 126.6636 94.2176) (end 126.6636 87.2556) (width 0.25) (layer F.Cu) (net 13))
 (segment (start 126.6636 87.2556) (end 124.748 85.34) (width 0.25) (layer F.Cu) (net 13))
 (segment (start 133.498 98.865) (end 132.3227 98.865) (width 0.25) (layer F.Cu) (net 13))
 (segment (start 133.498 98.865) (end 136.038 98.865) (width 0.25) (layer B.Cu) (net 13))
 (segment (start 125.038 98.865) (end 123.8627 98.865) (width 0.25) (layer F.Cu) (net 11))
 (segment (start 122.498 98.3899) (end 123.3876 98.3899) (width 0.25) (layer F.Cu) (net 11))
 (segment (start 123.3876 98.3899) (end 123.8627 98.865) (width 0.25) (layer F.Cu) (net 11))
 (segment (start 122.498 98.3899) (end 122.498 97.6897) (width 0.25) (layer F.Cu) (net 11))
 (segment (start 122.498 98.865) (end 122.498 98.3899) (width 0.25) (layer F.Cu) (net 11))
 (segment (start 122.498 97.6897) (end 121.9104 97.6897) (width 0.25) (layer F.Cu) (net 11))
 (segment (start 121.9104 97.6897) (end 119.748 95.5273) (width 0.25) (layer F.Cu) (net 11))
 (segment (start 119.748 95.5273) (end 119.748 85.3525) (width 0.25) (layer F.Cu) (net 11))
 (segment (start 127.998 101.615) (end 126.8227 101.615) (width 0.25) (layer F.Cu) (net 9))
 (segment (start 126.8227 101.615) (end 125.6474 100.4397) (width 0.25) (layer F.Cu) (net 9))
 (segment (start 125.6474 100.4397) (end 121.8929 100.4397) (width 0.25) (layer F.Cu) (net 9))
 (segment (start 121.8929 100.4397) (end 114.498 93.0448) (width 0.25) (layer F.Cu) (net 9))
 (segment (start 114.498 93.0448) (end 114.498 85.34) (width 0.25) (layer F.Cu) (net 9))
 (segment (start 130.538 101.615) (end 127.998 101.615) (width 0.25) (layer B.Cu) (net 9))
 (segment (start 133.498 104.365) (end 133.498 105.5403) (width 0.25) (layer F.Cu) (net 6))
 (segment (start 133.498 105.5403) (end 134.0856 105.5403) (width 0.25) (layer F.Cu) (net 6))
 (segment (start 134.0856 105.5403) (end 134.6734 106.1281) (width 0.25) (layer F.Cu) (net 6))
 (segment (start 134.6734 106.1281) (end 134.6734 113.9391) (width 0.25) (layer F.Cu) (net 6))
 (segment (start 134.6734 113.9391) (end 133.748 114.8645) (width 0.25) (layer F.Cu) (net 6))
 (segment (start 133.498 104.365) (end 136.038 104.365) (width 0.25) (layer B.Cu) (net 6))
 (segment (start 125.038 104.365) (end 125.038 105.5403) (width 0.25) (layer F.Cu) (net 4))
 (segment (start 125.038 105.5403) (end 125.185 105.5403) (width 0.25) (layer F.Cu) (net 4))
 (segment (start 125.185 105.5403) (end 126.2133 106.5686) (width 0.25) (layer F.Cu) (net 4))
 (segment (start 126.2133 106.5686) (end 126.2133 109.2338) (width 0.25) (layer F.Cu) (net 4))
 (segment (start 126.2133 109.2338) (end 132.8839 115.9044) (width 0.25) (layer F.Cu) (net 4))
 (segment (start 132.8839 115.9044) (end 137.7211 115.9044) (width 0.25) (layer F.Cu) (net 4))
 (segment (start 137.7211 115.9044) (end 138.748 114.8775) (width 0.25) (layer F.Cu) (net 4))
 (segment (start 122.498 104.365) (end 125.038 104.365) (width 0.25) (layer B.Cu) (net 4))
 (segment (start 130.538 107.115) (end 130.538 105.9397) (width 0.25) (layer F.Cu) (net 2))
 (segment (start 130.538 105.9397) (end 130.685 105.9397) (width 0.25) (layer F.Cu) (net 2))
 (segment (start 130.685 105.9397) (end 131.7133 104.9114) (width 0.25) (layer F.Cu) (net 2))
 (segment (start 131.7133 104.9114) (end 131.7133 103.9646) (width 0.25) (layer F.Cu) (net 2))
 (segment (start 131.7133 103.9646) (end 132.4883 103.1896) (width 0.25) (layer F.Cu) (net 2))
 (segment (start 132.4883 103.1896) (end 134.5291 103.1896) (width 0.25) (layer F.Cu) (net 2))
 (segment (start 134.5291 103.1896) (end 134.6734 103.3339) (width 0.25) (layer F.Cu) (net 2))
 (segment (start 134.6734 103.3339) (end 134.6734 104.7062) (width 0.25) (layer F.Cu) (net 2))
 (segment (start 134.6734 104.7062) (end 135.7072 105.74) (width 0.25) (layer F.Cu) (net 2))
 (segment (start 135.7072 105.74) (end 136.3501 105.74) (width 0.25) (layer F.Cu) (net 2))
 (segment (start 136.3501 105.74) (end 143.998 113.3879) (width 0.25) (layer F.Cu) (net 2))
 (segment (start 143.998 113.3879) (end 143.998 114.8775) (width 0.25) (layer F.Cu) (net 2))
 (segment (start 127.998 107.115) (end 130.538 107.115) (width 0.25) (layer F.Cu) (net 2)))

